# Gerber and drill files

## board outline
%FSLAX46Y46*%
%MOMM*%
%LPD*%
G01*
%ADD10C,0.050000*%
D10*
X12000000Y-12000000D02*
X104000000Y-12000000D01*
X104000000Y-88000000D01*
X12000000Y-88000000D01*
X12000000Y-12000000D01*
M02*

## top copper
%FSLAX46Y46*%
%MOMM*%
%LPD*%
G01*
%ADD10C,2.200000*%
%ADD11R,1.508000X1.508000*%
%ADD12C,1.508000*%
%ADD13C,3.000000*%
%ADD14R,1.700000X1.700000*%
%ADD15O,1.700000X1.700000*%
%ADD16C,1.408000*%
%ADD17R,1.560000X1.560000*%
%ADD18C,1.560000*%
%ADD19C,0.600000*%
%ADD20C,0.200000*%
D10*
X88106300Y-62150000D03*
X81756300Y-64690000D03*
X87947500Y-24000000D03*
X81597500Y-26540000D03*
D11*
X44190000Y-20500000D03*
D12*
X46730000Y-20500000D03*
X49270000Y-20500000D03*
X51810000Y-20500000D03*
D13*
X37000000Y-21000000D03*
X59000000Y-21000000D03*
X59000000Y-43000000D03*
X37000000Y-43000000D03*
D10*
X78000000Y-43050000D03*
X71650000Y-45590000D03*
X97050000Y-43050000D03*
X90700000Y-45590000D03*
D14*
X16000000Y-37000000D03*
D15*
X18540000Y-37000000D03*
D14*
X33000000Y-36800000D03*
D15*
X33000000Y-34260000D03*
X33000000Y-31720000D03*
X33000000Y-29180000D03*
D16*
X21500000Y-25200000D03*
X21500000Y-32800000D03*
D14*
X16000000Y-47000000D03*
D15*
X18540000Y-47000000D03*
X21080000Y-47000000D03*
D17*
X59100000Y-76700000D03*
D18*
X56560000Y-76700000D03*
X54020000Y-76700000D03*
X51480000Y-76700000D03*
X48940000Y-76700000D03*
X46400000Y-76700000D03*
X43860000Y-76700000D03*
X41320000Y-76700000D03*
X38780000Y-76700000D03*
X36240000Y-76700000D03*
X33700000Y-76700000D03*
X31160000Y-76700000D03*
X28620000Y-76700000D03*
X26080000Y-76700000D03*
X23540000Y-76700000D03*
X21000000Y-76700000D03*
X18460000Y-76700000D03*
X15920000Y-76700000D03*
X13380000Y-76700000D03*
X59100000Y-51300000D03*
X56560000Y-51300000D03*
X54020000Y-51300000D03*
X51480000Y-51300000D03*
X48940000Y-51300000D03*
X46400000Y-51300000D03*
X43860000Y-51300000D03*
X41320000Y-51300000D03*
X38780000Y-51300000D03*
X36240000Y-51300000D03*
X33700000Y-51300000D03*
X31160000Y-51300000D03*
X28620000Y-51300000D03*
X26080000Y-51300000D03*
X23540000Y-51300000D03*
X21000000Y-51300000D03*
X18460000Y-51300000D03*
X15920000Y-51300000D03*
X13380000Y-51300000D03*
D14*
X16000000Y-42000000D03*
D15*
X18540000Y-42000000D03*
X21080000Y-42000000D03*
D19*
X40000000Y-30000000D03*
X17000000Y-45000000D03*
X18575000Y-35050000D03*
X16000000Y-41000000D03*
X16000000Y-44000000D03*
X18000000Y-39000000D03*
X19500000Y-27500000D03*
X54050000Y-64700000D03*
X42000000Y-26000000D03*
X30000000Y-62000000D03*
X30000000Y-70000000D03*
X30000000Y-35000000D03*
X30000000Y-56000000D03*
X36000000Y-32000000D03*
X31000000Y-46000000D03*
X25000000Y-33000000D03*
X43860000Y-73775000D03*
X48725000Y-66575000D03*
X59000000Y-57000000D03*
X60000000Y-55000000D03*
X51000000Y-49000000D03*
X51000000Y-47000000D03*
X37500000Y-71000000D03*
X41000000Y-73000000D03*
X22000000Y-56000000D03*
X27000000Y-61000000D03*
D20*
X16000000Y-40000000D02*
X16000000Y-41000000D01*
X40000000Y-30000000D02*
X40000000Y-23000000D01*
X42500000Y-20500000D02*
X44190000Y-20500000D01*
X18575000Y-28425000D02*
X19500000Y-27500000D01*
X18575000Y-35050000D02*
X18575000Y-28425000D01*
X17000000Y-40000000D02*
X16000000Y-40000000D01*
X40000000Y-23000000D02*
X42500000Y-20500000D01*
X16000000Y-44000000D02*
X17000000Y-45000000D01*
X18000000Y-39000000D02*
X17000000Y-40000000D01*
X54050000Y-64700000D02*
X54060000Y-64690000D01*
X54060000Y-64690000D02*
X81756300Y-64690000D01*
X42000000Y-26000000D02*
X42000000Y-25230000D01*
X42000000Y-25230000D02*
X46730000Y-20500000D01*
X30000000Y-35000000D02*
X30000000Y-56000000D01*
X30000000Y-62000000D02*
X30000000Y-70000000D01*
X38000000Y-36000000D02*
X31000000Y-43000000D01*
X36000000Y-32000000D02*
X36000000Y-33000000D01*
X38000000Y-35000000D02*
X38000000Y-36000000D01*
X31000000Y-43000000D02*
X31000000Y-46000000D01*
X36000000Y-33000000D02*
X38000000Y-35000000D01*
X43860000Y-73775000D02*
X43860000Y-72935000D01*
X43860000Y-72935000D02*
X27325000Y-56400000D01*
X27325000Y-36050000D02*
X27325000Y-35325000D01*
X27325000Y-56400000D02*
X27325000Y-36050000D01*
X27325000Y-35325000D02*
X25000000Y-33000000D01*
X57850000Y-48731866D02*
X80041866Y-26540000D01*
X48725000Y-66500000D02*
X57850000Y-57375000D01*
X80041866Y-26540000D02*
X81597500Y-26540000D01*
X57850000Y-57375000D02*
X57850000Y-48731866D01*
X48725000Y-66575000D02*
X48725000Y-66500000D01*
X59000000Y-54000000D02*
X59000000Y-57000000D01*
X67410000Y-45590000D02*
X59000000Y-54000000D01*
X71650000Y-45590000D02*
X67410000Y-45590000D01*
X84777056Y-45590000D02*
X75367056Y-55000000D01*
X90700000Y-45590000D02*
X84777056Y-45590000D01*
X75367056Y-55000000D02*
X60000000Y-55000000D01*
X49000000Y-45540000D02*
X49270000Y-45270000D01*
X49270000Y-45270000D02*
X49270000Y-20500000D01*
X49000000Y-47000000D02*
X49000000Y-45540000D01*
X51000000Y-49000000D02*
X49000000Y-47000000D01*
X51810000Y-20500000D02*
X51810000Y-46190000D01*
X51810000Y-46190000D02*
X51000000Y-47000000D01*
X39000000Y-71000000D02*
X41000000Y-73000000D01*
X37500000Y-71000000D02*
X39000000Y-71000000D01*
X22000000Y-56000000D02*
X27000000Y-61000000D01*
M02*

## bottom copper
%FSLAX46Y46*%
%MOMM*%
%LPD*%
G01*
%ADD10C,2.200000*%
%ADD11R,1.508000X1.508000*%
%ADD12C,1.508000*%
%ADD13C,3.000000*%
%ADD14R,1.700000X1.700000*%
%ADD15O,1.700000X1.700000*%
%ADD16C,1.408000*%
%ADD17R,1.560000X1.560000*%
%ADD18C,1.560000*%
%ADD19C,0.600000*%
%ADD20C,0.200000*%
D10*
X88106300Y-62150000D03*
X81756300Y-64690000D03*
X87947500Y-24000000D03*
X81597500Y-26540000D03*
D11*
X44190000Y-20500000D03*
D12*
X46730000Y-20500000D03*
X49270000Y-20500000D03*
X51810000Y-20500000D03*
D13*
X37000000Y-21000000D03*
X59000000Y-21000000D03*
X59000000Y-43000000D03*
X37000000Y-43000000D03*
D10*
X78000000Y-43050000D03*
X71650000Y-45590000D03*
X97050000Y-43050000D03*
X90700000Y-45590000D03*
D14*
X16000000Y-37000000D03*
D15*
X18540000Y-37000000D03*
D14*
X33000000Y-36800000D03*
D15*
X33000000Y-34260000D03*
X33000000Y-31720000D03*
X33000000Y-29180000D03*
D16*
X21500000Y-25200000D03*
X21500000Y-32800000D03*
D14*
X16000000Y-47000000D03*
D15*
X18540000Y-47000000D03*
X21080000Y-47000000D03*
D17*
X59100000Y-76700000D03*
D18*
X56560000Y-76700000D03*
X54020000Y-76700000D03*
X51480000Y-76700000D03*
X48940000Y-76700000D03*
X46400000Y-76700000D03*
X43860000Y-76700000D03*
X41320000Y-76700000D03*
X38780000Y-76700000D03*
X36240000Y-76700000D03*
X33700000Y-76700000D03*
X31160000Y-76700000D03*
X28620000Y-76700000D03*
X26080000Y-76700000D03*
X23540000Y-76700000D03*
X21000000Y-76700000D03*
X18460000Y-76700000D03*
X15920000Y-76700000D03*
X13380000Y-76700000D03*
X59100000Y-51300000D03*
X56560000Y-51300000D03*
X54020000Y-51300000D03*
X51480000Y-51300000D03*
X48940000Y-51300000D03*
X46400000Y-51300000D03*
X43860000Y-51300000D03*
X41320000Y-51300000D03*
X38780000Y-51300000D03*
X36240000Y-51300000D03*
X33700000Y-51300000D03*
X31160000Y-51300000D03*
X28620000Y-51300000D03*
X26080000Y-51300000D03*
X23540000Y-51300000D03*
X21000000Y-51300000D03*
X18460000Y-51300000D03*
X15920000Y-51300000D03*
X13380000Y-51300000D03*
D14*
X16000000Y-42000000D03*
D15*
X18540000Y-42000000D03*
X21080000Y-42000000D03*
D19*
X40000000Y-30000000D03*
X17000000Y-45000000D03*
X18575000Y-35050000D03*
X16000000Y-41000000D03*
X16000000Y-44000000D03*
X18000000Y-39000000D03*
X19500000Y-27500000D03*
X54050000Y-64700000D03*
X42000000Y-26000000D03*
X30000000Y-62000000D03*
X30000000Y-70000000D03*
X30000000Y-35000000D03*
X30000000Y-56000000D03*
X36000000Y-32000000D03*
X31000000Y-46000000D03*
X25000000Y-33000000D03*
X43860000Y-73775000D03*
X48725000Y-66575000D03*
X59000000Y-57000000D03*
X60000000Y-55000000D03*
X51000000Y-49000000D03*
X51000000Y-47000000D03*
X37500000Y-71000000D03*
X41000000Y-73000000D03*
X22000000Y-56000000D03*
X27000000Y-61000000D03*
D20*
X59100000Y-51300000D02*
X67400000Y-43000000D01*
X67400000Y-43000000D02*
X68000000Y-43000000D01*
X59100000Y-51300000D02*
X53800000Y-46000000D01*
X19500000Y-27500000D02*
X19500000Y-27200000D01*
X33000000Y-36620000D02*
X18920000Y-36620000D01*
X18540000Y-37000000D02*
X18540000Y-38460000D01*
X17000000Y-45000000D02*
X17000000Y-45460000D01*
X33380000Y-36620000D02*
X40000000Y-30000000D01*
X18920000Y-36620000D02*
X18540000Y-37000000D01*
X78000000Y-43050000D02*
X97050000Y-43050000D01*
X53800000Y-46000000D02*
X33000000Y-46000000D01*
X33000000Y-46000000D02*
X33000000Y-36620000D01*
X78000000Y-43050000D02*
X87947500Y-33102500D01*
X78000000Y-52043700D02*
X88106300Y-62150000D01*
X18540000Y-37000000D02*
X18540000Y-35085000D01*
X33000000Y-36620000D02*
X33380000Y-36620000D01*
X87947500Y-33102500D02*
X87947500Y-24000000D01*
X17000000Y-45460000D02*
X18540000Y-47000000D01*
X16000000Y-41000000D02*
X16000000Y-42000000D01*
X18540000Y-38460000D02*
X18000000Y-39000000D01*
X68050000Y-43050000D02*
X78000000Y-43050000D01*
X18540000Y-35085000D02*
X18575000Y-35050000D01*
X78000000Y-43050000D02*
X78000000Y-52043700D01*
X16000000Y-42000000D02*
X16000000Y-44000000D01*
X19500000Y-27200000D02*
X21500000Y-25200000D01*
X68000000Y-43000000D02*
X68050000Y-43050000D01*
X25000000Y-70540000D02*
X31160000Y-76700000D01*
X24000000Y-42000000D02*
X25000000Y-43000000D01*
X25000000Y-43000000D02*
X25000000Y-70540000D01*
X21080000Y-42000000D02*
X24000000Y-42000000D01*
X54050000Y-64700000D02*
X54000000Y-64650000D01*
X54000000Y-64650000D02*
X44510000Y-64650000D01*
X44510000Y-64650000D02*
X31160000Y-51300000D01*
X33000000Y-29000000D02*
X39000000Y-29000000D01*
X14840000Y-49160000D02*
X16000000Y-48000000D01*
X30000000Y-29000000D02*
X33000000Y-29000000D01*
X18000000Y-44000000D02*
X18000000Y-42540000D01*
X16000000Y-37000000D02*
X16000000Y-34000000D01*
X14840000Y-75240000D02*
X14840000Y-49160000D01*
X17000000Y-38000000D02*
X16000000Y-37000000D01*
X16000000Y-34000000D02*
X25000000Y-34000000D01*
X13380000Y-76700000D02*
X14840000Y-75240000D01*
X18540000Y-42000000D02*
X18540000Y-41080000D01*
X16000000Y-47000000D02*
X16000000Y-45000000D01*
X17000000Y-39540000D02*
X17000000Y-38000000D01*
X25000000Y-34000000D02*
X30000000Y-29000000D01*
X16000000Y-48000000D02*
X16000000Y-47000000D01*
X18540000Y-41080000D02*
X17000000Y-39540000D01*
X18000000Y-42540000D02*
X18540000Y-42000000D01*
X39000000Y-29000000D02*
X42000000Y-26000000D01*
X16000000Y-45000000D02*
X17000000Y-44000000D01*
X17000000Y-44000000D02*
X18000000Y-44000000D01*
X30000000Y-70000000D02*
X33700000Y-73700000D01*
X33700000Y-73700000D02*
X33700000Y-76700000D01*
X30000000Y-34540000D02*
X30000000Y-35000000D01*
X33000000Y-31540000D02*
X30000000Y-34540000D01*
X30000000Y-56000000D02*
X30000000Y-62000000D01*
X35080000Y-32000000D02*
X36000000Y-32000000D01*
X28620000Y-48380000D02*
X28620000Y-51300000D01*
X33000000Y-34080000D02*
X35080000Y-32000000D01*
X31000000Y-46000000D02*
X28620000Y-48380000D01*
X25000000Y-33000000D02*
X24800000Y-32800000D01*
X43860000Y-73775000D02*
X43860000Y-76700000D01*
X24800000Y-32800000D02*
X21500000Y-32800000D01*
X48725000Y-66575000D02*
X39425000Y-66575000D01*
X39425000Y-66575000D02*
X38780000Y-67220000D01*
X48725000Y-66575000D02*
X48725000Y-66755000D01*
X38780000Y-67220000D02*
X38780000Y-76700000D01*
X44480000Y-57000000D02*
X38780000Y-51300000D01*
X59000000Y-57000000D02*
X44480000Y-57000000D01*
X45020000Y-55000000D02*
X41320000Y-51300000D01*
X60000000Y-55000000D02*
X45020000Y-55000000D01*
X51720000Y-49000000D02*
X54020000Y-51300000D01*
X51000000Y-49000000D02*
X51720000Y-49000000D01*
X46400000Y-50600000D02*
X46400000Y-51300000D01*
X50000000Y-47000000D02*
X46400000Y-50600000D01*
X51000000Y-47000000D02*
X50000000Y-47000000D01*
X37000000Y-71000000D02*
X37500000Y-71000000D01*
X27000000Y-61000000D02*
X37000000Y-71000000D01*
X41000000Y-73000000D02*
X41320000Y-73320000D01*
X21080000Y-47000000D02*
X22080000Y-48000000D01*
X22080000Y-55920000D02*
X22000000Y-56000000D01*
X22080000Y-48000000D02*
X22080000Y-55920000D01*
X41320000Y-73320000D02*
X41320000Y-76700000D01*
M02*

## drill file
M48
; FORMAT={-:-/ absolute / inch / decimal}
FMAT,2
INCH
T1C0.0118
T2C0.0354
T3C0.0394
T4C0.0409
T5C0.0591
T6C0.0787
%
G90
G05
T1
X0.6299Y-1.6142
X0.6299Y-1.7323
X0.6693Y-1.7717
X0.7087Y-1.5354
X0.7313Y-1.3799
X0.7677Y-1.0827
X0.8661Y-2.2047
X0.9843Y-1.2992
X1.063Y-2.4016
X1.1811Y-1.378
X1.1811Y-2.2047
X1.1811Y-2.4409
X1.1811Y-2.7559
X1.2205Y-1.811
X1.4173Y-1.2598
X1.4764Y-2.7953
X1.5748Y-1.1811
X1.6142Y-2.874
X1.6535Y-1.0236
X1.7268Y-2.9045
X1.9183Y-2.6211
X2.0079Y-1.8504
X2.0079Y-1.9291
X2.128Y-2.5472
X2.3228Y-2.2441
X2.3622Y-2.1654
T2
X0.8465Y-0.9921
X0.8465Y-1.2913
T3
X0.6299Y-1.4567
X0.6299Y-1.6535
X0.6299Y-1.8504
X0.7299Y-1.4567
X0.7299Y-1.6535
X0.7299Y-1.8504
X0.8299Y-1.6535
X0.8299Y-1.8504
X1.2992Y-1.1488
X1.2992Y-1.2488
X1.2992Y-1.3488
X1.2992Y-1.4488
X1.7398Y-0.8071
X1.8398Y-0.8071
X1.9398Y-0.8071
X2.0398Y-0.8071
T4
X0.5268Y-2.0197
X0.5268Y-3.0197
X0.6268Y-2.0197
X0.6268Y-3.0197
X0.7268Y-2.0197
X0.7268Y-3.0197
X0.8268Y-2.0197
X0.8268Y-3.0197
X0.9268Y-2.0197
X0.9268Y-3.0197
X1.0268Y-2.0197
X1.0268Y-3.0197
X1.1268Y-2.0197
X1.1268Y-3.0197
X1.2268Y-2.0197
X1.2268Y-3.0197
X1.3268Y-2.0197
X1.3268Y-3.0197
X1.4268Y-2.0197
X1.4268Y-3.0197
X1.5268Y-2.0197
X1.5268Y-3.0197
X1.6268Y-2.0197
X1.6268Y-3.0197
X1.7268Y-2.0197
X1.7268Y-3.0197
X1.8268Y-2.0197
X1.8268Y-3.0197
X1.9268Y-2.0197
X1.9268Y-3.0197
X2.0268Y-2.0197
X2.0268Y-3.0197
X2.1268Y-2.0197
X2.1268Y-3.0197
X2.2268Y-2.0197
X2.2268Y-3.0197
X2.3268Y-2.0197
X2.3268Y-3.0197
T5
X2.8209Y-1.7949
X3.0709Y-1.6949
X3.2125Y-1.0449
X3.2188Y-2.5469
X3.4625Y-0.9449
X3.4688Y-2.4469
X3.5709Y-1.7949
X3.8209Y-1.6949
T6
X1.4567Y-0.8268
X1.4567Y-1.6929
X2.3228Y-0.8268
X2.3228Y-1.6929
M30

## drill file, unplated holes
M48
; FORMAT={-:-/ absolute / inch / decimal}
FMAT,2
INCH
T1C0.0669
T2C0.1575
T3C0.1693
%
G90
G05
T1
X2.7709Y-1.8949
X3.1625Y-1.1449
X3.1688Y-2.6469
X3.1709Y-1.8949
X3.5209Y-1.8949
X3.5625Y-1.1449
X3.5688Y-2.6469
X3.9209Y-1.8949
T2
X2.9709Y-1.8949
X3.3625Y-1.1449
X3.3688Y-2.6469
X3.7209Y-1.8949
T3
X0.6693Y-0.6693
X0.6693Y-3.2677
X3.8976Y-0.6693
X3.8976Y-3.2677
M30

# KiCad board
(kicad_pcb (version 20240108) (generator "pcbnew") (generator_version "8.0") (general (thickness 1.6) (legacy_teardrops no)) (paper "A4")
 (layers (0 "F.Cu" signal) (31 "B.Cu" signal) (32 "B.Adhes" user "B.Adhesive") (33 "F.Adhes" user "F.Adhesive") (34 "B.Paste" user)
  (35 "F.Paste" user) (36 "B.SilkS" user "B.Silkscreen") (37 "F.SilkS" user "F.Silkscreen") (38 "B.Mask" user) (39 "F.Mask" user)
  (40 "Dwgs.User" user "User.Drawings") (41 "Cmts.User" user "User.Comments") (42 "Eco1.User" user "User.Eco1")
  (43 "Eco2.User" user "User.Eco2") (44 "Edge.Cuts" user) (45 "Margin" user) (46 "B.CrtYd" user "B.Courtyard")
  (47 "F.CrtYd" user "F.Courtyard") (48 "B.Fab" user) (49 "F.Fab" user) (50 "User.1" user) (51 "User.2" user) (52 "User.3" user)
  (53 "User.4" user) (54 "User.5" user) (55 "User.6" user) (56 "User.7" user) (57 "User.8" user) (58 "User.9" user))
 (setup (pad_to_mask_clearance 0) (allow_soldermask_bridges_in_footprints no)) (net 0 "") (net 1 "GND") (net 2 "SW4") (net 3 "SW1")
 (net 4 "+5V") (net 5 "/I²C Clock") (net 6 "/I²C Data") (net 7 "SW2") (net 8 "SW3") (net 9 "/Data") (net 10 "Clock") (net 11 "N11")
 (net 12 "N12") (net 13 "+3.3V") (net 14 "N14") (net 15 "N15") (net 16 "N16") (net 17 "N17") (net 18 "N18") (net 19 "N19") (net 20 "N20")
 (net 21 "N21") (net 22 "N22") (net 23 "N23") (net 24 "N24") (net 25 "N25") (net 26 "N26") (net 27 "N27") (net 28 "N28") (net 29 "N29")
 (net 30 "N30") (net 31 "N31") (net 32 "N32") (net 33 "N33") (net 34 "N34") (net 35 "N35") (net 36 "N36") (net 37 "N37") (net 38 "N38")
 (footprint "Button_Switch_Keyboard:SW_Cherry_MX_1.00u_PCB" (layer "F.Cu") (at 88.1063 62.15)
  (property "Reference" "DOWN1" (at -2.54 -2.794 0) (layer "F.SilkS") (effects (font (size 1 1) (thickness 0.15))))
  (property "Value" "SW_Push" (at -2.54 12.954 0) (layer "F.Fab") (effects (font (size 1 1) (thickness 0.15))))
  (pad "" np_thru_hole circle (at -7.62 5.08) (size 1.7 1.7) (drill 1.7) (layers "*.Cu" "*.Mask"))
  (pad "" np_thru_hole circle (at -2.54 5.08) (size 4 4) (drill 4) (layers "*.Cu" "*.Mask"))
  (pad "" np_thru_hole circle (at 2.54 5.08) (size 1.7 1.7) (drill 1.7) (layers "*.Cu" "*.Mask"))
  (pad "1" thru_hole circle (at 0 0) (size 2.2 2.2) (drill 1.5) (layers "*.Cu" "*.Mask") (remove_unused_layers no) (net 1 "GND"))
  (pad "2" thru_hole circle (at -6.35 2.54) (size 2.2 2.2) (drill 1.5) (layers "*.Cu" "*.Mask") (remove_unused_layers no) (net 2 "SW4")))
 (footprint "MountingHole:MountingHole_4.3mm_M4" (layer "F.Cu") (at 99 17)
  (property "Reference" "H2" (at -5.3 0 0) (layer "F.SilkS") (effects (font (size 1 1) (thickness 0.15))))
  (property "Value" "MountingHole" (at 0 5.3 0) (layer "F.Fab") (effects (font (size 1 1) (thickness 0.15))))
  (pad "" np_thru_hole circle (at 0 0) (size 4.3 4.3) (drill 4.3) (layers "*.Cu" "*.Mask")))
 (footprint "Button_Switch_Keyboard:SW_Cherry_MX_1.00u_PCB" (layer "F.Cu") (at 87.9475 24)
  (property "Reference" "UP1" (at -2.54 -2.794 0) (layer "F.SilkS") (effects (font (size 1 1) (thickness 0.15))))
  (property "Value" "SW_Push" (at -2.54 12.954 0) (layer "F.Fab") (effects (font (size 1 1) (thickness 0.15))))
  (pad "" np_thru_hole circle (at -7.62 5.08) (size 1.7 1.7) (drill 1.7) (layers "*.Cu" "*.Mask"))
  (pad "" np_thru_hole circle (at -2.54 5.08) (size 4 4) (drill 4) (layers "*.Cu" "*.Mask"))
  (pad "" np_thru_hole circle (at 2.54 5.08) (size 1.7 1.7) (drill 1.7) (layers "*.Cu" "*.Mask"))
  (pad "1" thru_hole circle (at 0 0) (size 2.2 2.2) (drill 1.5) (layers "*.Cu" "*.Mask") (remove_unused_layers no) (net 1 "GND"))
  (pad "2" thru_hole circle (at -6.35 2.54) (size 2.2 2.2) (drill 1.5) (layers "*.Cu" "*.Mask") (remove_unused_layers no) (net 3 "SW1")))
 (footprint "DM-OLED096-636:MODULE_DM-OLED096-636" (layer "F.Cu") (at 48 32)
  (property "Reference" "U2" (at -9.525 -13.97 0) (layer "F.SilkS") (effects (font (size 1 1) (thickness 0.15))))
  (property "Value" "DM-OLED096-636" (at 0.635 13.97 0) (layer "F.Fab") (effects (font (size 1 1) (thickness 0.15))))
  (pad "1" thru_hole rect (at -3.81 -11.5) (size 1.508 1.508) (drill 1) (layers "*.Cu" "*.Mask") (remove_unused_layers no) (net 1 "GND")
   (solder_mask_margin 0.102))
  (pad "2" thru_hole circle (at -1.27 -11.5) (size 1.508 1.508) (drill 1) (layers "*.Cu" "*.Mask") (remove_unused_layers no) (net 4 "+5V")
   (solder_mask_margin 0.102))
  (pad "3" thru_hole circle (at 1.27 -11.5) (size 1.508 1.508) (drill 1) (layers "*.Cu" "*.Mask") (remove_unused_layers no)
   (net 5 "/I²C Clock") (solder_mask_margin 0.102))
  (pad "4" thru_hole circle (at 3.81 -11.5) (size 1.508 1.508) (drill 1) (layers "*.Cu" "*.Mask") (remove_unused_layers no)
   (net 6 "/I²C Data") (solder_mask_margin 0.102))
  (pad "S1" thru_hole circle (at -11 -11) (size 3 3) (drill 2) (layers "*.Cu" "*.Mask") (remove_unused_layers no) (solder_mask_margin 0.102))
  (pad "S2" thru_hole circle (at 11 -11) (size 3 3) (drill 2) (layers "*.Cu" "*.Mask") (remove_unused_layers no) (solder_mask_margin 0.102))
  (pad "S3" thru_hole circle (at 11 11) (size 3 3) (drill 2) (layers "*.Cu" "*.Mask") (remove_unused_layers no) (solder_mask_margin 0.102))
  (pad "S4" thru_hole circle (at -11 11) (size 3 3) (drill 2) (layers "*.Cu" "*.Mask") (remove_unused_layers no) (solder_mask_margin 0.102)))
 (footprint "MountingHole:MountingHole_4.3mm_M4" (layer "F.Cu") (at 99 83)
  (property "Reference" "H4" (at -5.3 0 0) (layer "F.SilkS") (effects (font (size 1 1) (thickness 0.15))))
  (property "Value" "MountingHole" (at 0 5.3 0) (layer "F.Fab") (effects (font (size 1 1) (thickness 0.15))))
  (pad "" np_thru_hole circle (at 0 0) (size 4.3 4.3) (drill 4.3) (layers "*.Cu" "*.Mask")))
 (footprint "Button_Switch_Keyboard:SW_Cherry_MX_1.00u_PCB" (layer "F.Cu") (at 78 43.05)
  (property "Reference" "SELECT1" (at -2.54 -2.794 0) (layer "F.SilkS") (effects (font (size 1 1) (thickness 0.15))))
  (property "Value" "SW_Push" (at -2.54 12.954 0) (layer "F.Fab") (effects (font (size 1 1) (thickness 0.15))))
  (pad "" np_thru_hole circle (at -7.62 5.08) (size 1.7 1.7) (drill 1.7) (layers "*.Cu" "*.Mask"))
  (pad "" np_thru_hole circle (at -2.54 5.08) (size 4 4) (drill 4) (layers "*.Cu" "*.Mask"))
  (pad "" np_thru_hole circle (at 2.54 5.08) (size 1.7 1.7) (drill 1.7) (layers "*.Cu" "*.Mask"))
  (pad "1" thru_hole circle (at 0 0) (size 2.2 2.2) (drill 1.5) (layers "*.Cu" "*.Mask") (remove_unused_layers no) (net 1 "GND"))
  (pad "2" thru_hole circle (at -6.35 2.54) (size 2.2 2.2) (drill 1.5) (layers "*.Cu" "*.Mask") (remove_unused_layers no) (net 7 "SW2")))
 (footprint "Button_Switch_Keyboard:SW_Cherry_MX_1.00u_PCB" (layer "F.Cu") (at 97.05 43.05)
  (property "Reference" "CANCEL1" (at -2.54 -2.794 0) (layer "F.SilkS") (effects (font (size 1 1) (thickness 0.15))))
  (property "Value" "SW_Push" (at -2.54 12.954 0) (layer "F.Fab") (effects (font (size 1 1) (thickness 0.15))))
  (pad "" np_thru_hole circle (at -7.62 5.08) (size 1.7 1.7) (drill 1.7) (layers "*.Cu" "*.Mask"))
  (pad "" np_thru_hole circle (at -2.54 5.08) (size 4 4) (drill 4) (layers "*.Cu" "*.Mask"))
  (pad "" np_thru_hole circle (at 2.54 5.08) (size 1.7 1.7) (drill 1.7) (layers "*.Cu" "*.Mask"))
  (pad "1" thru_hole circle (at 0 0) (size 2.2 2.2) (drill 1.5) (layers "*.Cu" "*.Mask") (remove_unused_layers no) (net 1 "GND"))
  (pad "2" thru_hole circle (at -6.35 2.54) (size 2.2 2.2) (drill 1.5) (layers "*.Cu" "*.Mask") (remove_unused_layers no) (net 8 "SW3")))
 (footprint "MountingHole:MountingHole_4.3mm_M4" (layer "F.Cu") (at 17 17)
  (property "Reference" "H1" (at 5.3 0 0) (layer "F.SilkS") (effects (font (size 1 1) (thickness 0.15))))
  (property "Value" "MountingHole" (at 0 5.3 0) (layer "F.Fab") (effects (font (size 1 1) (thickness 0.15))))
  (pad "" np_thru_hole circle (at 0 0) (size 4.3 4.3) (drill 4.3) (layers "*.Cu" "*.Mask")))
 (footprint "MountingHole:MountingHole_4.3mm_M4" (layer "F.Cu") (at 17 83)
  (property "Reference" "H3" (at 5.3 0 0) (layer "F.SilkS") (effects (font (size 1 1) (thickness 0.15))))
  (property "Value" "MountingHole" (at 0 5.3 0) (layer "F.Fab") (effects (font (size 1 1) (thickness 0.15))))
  (pad "" np_thru_hole circle (at 0 0) (size 4.3 4.3) (drill 4.3) (layers "*.Cu" "*.Mask")))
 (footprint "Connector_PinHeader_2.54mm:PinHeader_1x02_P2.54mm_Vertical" (layer "B.Cu") (at 16 37 -90)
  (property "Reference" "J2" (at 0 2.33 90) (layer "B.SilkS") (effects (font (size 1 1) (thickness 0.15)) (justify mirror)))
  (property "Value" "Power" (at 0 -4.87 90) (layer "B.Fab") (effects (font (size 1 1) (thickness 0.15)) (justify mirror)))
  (pad "1" thru_hole rect (at 0 0 270) (size 1.7 1.7) (drill 1) (layers "*.Cu" "*.Mask") (remove_unused_layers no) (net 4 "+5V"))
  (pad "2" thru_hole oval (at 0 -2.54 270) (size 1.7 1.7) (drill 1) (layers "*.Cu" "*.Mask") (remove_unused_layers no) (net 1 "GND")))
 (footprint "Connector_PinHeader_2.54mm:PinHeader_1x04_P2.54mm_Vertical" (layer "B.Cu") (at 33 36.8)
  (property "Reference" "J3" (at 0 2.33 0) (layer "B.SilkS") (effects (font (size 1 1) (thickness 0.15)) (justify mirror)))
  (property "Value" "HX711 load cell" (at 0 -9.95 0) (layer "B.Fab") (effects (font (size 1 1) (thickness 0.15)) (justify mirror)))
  (pad "1" thru_hole rect (at 0 0) (size 1.7 1.7) (drill 1) (layers "*.Cu" "*.Mask") (remove_unused_layers no) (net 1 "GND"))
  (pad "2" thru_hole oval (at 0 -2.54) (size 1.7 1.7) (drill 1) (layers "*.Cu" "*.Mask") (remove_unused_layers no) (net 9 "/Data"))
  (pad "3" thru_hole oval (at 0 -5.08) (size 1.7 1.7) (drill 1) (layers "*.Cu" "*.Mask") (remove_unused_layers no) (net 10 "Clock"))
  (pad "4" thru_hole oval (at 0 -7.62) (size 1.7 1.7) (drill 1) (layers "*.Cu" "*.Mask") (remove_unused_layers no) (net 4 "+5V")))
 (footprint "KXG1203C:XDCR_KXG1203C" (layer "B.Cu") (at 21.5 29 90)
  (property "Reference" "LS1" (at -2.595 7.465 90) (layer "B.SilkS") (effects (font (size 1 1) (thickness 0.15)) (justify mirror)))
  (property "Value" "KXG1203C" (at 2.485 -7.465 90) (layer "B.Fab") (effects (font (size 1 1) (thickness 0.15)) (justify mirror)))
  (pad "N" thru_hole circle (at 3.8 0 90) (size 1.408 1.408) (drill 0.9) (layers "*.Cu" "*.Mask") (remove_unused_layers no) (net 1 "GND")
   (solder_mask_margin 0.102))
  (pad "P" thru_hole circle (at -3.8 0 90) (size 1.408 1.408) (drill 0.9) (layers "*.Cu" "*.Mask") (remove_unused_layers no) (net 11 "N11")
   (solder_mask_margin 0.102)))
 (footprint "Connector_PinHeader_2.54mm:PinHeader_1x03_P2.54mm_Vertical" (layer "B.Cu") (at 16 47 -90)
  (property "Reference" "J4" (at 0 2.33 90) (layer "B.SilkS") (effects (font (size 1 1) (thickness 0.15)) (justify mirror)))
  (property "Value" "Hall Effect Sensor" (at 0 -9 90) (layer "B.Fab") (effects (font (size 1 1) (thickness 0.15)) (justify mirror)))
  (pad "1" thru_hole rect (at 0 0 270) (size 1.7 1.7) (drill 1) (layers "*.Cu" "*.Mask") (remove_unused_layers no) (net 4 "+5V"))
  (pad "2" thru_hole oval (at 0 -2.54 270) (size 1.7 1.7) (drill 1) (layers "*.Cu" "*.Mask") (remove_unused_layers no) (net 1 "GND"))
  (pad "3" thru_hole oval (at 0 -5.08 270) (size 1.7 1.7) (drill 1) (layers "*.Cu" "*.Mask") (remove_unused_layers no) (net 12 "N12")))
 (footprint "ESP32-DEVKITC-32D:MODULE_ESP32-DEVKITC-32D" (layer "B.Cu") (at 39.34 64 90)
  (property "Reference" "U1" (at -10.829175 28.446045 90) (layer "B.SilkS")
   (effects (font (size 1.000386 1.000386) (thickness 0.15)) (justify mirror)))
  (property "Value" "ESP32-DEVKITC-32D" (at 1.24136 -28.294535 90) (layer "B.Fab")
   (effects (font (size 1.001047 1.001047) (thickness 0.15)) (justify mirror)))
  (pad "J2-1" thru_hole rect (at -12.7 19.76 90) (size 1.56 1.56) (drill 1.04) (layers "*.Cu" "*.Mask") (remove_unused_layers no)
   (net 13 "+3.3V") (solder_mask_margin 0.102))
  (pad "J2-2" thru_hole circle (at -12.7 17.22 90) (size 1.56 1.56) (drill 1.04) (layers "*.Cu" "*.Mask") (remove_unused_layers no)
   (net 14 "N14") (solder_mask_margin 0.102))
  (pad "J2-3" thru_hole circle (at -12.7 14.68 90) (size 1.56 1.56) (drill 1.04) (layers "*.Cu" "*.Mask") (remove_unused_layers no)
   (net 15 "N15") (solder_mask_margin 0.102))
  (pad "J2-4" thru_hole circle (at -12.7 12.14 90) (size 1.56 1.56) (drill 1.04) (layers "*.Cu" "*.Mask") (remove_unused_layers no)
   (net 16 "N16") (solder_mask_margin 0.102))
  (pad "J2-5" thru_hole circle (at -12.7 9.6 90) (size 1.56 1.56) (drill 1.04) (layers "*.Cu" "*.Mask") (remove_unused_layers no)
   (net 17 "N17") (solder_mask_margin 0.102))
  (pad "J2-6" thru_hole circle (at -12.7 7.06 90) (size 1.56 1.56) (drill 1.04) (layers "*.Cu" "*.Mask") (remove_unused_layers no)
   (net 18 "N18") (solder_mask_margin 0.102))
  (pad "J2-7" thru_hole circle (at -12.7 4.52 90) (size 1.56 1.56) (drill 1.04) (layers "*.Cu" "*.Mask") (remove_unused_layers no)
   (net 11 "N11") (solder_mask_margin 0.102))
  (pad "J2-8" thru_hole circle (at -12.7 1.98 90) (size 1.56 1.56) (drill 1.04) (layers "*.Cu" "*.Mask") (remove_unused_layers no)
   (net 12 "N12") (solder_mask_margin 0.102))
  (pad "J2-9" thru_hole circle (at -12.7 -0.56 90) (size 1.56 1.56) (drill 1.04) (layers "*.Cu" "*.Mask") (remove_unused_layers no)
   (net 3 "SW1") (solder_mask_margin 0.102))
  (pad "J2-10" thru_hole circle (at -12.7 -3.1 90) (size 1.56 1.56) (drill 1.04) (layers "*.Cu" "*.Mask") (remove_unused_layers no)
   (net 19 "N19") (solder_mask_margin 0.102))
  (pad "J2-11" thru_hole circle (at -12.7 -5.64 90) (size 1.56 1.56) (drill 1.04) (layers "*.Cu" "*.Mask") (remove_unused_layers no)
   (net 10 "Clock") (solder_mask_margin 0.102))
  (pad "J2-12" thru_hole circle (at -12.7 -8.18 90) (size 1.56 1.56) (drill 1.04) (layers "*.Cu" "*.Mask") (remove_unused_layers no)
   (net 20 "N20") (solder_mask_margin 0.102))
  (pad "J2-13" thru_hole circle (at -12.7 -10.72 90) (size 1.56 1.56) (drill 1.04) (layers "*.Cu" "*.Mask") (remove_unused_layers no)
   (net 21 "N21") (solder_mask_margin 0.102))
  (pad "J2-14" thru_hole circle (at -12.7 -13.26 90) (size 1.56 1.56) (drill 1.04) (layers "*.Cu" "*.Mask") (remove_unused_layers no)
   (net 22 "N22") (solder_mask_margin 0.102))
  (pad "J2-15" thru_hole circle (at -12.7 -15.8 90) (size 1.56 1.56) (drill 1.04) (layers "*.Cu" "*.Mask") (remove_unused_layers no)
   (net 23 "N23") (solder_mask_margin 0.102))
  (pad "J2-16" thru_hole circle (at -12.7 -18.34 90) (size 1.56 1.56) (drill 1.04) (layers "*.Cu" "*.Mask") (remove_unused_layers no)
   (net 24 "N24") (solder_mask_margin 0.102))
  (pad "J2-17" thru_hole circle (at -12.7 -20.88 90) (size 1.56 1.56) (drill 1.04) (layers "*.Cu" "*.Mask") (remove_unused_layers no)
   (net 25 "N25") (solder_mask_margin 0.102))
  (pad "J2-18" thru_hole circle (at -12.7 -23.42 90) (size 1.56 1.56) (drill 1.04) (layers "*.Cu" "*.Mask") (remove_unused_layers no)
   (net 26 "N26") (solder_mask_margin 0.102))
  (pad "J2-19" thru_hole circle (at -12.7 -25.96 90) (size 1.56 1.56) (drill 1.04) (layers "*.Cu" "*.Mask") (remove_unused_layers no)
   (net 4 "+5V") (solder_mask_margin 0.102))
  (pad "J3-1" thru_hole circle (at 12.7 19.76 90) (size 1.56 1.56) (drill 1.04) (layers "*.Cu" "*.Mask") (remove_unused_layers no)
   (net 1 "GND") (solder_mask_margin 0.102))
  (pad "J3-2" thru_hole circle (at 12.7 17.22 90) (size 1.56 1.56) (drill 1.04) (layers "*.Cu" "*.Mask") (remove_unused_layers no)
   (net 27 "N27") (solder_mask_margin 0.102))
  (pad "J3-3" thru_hole circle (at 12.7 14.68 90) (size 1.56 1.56) (drill 1.04) (layers "*.Cu" "*.Mask") (remove_unused_layers no)
   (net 5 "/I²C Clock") (solder_mask_margin 0.102))
  (pad "J3-4" thru_hole circle (at 12.7 12.14 90) (size 1.56 1.56) (drill 1.04) (layers "*.Cu" "*.Mask") (remove_unused_layers no)
   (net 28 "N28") (solder_mask_margin 0.102))
  (pad "J3-5" thru_hole circle (at 12.7 9.6 90) (size 1.56 1.56) (drill 1.04) (layers "*.Cu" "*.Mask") (remove_unused_layers no)
   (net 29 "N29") (solder_mask_margin 0.102))
  (pad "J3-6" thru_hole circle (at 12.7 7.06 90) (size 1.56 1.56) (drill 1.04) (layers "*.Cu" "*.Mask") (remove_unused_layers no)
   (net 6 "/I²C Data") (solder_mask_margin 0.102))
  (pad "J3-7" thru_hole circle (at 12.7 4.52 90) (size 1.56 1.56) (drill 1.04) (layers "*.Cu" "*.Mask") (remove_unused_layers no)
   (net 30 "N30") (solder_mask_margin 0.102))
  (pad "J3-8" thru_hole circle (at 12.7 1.98 90) (size 1.56 1.56) (drill 1.04) (layers "*.Cu" "*.Mask") (remove_unused_layers no)
   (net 8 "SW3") (solder_mask_margin 0.102))
  (pad "J3-9" thru_hole circle (at 12.7 -0.56 90) (size 1.56 1.56) (drill 1.04) (layers "*.Cu" "*.Mask") (remove_unused_layers no)
   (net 7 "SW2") (solder_mask_margin 0.102))
  (pad "J3-10" thru_hole circle (at 12.7 -3.1 90) (size 1.56 1.56) (drill 1.04) (layers "*.Cu" "*.Mask") (remove_unused_layers no)
   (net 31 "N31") (solder_mask_margin 0.102))
  (pad "J3-11" thru_hole circle (at 12.7 -5.64 90) (size 1.56 1.56) (drill 1.04) (layers "*.Cu" "*.Mask") (remove_unused_layers no)
   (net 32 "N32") (solder_mask_margin 0.102))
  (pad "J3-12" thru_hole circle (at 12.7 -8.18 90) (size 1.56 1.56) (drill 1.04) (layers "*.Cu" "*.Mask") (remove_unused_layers no)
   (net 2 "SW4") (solder_mask_margin 0.102))
  (pad "J3-13" thru_hole circle (at 12.7 -10.72 90) (size 1.56 1.56) (drill 1.04) (layers "*.Cu" "*.Mask") (remove_unused_layers no)
   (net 9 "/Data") (solder_mask_margin 0.102))
  (pad "J3-14" thru_hole circle (at 12.7 -13.26 90) (size 1.56 1.56) (drill 1.04) (layers "*.Cu" "*.Mask") (remove_unused_layers no)
   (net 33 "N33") (solder_mask_margin 0.102))
  (pad "J3-15" thru_hole circle (at 12.7 -15.8 90) (size 1.56 1.56) (drill 1.04) (layers "*.Cu" "*.Mask") (remove_unused_layers no)
   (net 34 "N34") (solder_mask_margin 0.102))
  (pad "J3-16" thru_hole circle (at 12.7 -18.34 90) (size 1.56 1.56) (drill 1.04) (layers "*.Cu" "*.Mask") (remove_unused_layers no)
   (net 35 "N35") (solder_mask_margin 0.102))
  (pad "J3-17" thru_hole circle (at 12.7 -20.88 90) (size 1.56 1.56) (drill 1.04) (layers "*.Cu" "*.Mask") (remove_unused_layers no)
   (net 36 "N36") (solder_mask_margin 0.102))
  (pad "J3-18" thru_hole circle (at 12.7 -23.42 90) (size 1.56 1.56) (drill 1.04) (layers "*.Cu" "*.Mask") (remove_unused_layers no)
   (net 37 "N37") (solder_mask_margin 0.102))
  (pad "J3-19" thru_hole circle (at 12.7 -25.96 90) (size 1.56 1.56) (drill 1.04) (layers "*.Cu" "*.Mask") (remove_unused_layers no)
   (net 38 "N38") (solder_mask_margin 0.102)))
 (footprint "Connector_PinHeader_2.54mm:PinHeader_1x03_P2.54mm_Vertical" (layer "B.Cu") (at 16 42 -90)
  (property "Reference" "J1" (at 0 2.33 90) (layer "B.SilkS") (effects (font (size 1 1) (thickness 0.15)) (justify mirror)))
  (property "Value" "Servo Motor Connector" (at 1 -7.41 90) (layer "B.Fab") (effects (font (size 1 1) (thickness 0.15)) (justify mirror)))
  (pad "1" thru_hole rect (at 0 0 270) (size 1.7 1.7) (drill 1) (layers "*.Cu" "*.Mask") (remove_unused_layers no) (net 1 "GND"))
  (pad "2" thru_hole oval (at 0 -2.54 270) (size 1.7 1.7) (drill 1) (layers "*.Cu" "*.Mask") (remove_unused_layers no) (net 4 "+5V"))
  (pad "3" thru_hole oval (at 0 -5.08 270) (size 1.7 1.7) (drill 1) (layers "*.Cu" "*.Mask") (remove_unused_layers no) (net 20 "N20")))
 (gr_rect (start 12 12) (end 104 88) (stroke (width 0.05) (type default)) (fill none) (layer "Edge.Cuts"))
 (segment (start 16 40) (end 16 41) (width 0.2) (layer "F.Cu") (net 1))
 (segment (start 40 30) (end 40 23) (width 0.2) (layer "F.Cu") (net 1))
 (segment (start 42.5 20.5) (end 44.19 20.5) (width 0.2) (layer "F.Cu") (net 1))
 (segment (start 18.575 28.425) (end 19.5 27.5) (width 0.2) (layer "F.Cu") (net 1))
 (segment (start 18.575 35.05) (end 18.575 28.425) (width 0.2) (layer "F.Cu") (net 1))
 (segment (start 17 40) (end 16 40) (width 0.2) (layer "F.Cu") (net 1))
 (segment (start 40 23) (end 42.5 20.5) (width 0.2) (layer "F.Cu") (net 1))
 (segment (start 16 44) (end 17 45) (width 0.2) (layer "F.Cu") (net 1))
 (segment (start 18 39) (end 17 40) (width 0.2) (layer "F.Cu") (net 1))
 (via (at 40 30) (size 0.6) (drill 0.3) (layers "F.Cu" "B.Cu") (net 1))
 (via (at 17 45) (size 0.6) (drill 0.3) (layers "F.Cu" "B.Cu") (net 1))
 (via (at 18.575 35.05) (size 0.6) (drill 0.3) (layers "F.Cu" "B.Cu") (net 1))
 (via (at 16 41) (size 0.6) (drill 0.3) (layers "F.Cu" "B.Cu") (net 1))
 (via (at 16 44) (size 0.6) (drill 0.3) (layers "F.Cu" "B.Cu") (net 1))
 (via (at 18 39) (size 0.6) (drill 0.3) (layers "F.Cu" "B.Cu") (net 1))
 (via (at 19.5 27.5) (size 0.6) (drill 0.3) (layers "F.Cu" "B.Cu") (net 1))
 (segment (start 59.1 51.3) (end 67.4 43) (width 0.2) (layer "B.Cu") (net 1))
 (segment (start 67.4 43) (end 68 43) (width 0.2) (layer "B.Cu") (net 1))
 (segment (start 59.1 51.3) (end 53.8 46) (width 0.2) (layer "B.Cu") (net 1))
 (segment (start 19.5 27.5) (end 19.5 27.2) (width 0.2) (layer "B.Cu") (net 1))
 (segment (start 33 36.62) (end 18.92 36.62) (width 0.2) (layer "B.Cu") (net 1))
 (segment (start 18.54 37) (end 18.54 38.46) (width 0.2) (layer "B.Cu") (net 1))
 (segment (start 17 45) (end 17 45.46) (width 0.2) (layer "B.Cu") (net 1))
 (segment (start 33.38 36.62) (end 40 30) (width 0.2) (layer "B.Cu") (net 1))
 (segment (start 18.92 36.62) (end 18.54 37) (width 0.2) (layer "B.Cu") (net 1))
 (segment (start 78 43.05) (end 97.05 43.05) (width 0.2) (layer "B.Cu") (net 1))
 (segment (start 53.8 46) (end 33 46) (width 0.2) (layer "B.Cu") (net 1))
 (segment (start 33 46) (end 33 36.62) (width 0.2) (layer "B.Cu") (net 1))
 (segment (start 78 43.05) (end 87.9475 33.1025) (width 0.2) (layer "B.Cu") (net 1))
 (segment (start 78 52.0437) (end 88.1063 62.15) (width 0.2) (layer "B.Cu") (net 1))
 (segment (start 18.54 37) (end 18.54 35.085) (width 0.2) (layer "B.Cu") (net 1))
 (segment (start 33 36.62) (end 33.38 36.62) (width 0.2) (layer "B.Cu") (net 1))
 (segment (start 87.9475 33.1025) (end 87.9475 24) (width 0.2) (layer "B.Cu") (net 1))
 (segment (start 17 45.46) (end 18.54 47) (width 0.2) (layer "B.Cu") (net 1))
 (segment (start 16 41) (end 16 42) (width 0.2) (layer "B.Cu") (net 1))
 (segment (start 18.54 38.46) (end 18 39) (width 0.2) (layer "B.Cu") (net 1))
 (segment (start 68.05 43.05) (end 78 43.05) (width 0.2) (layer "B.Cu") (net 1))
 (segment (start 18.54 35.085) (end 18.575 35.05) (width 0.2) (layer "B.Cu") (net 1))
 (segment (start 78 43.05) (end 78 52.0437) (width 0.2) (layer "B.Cu") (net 1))
 (segment (start 16 42) (end 16 44) (width 0.2) (layer "B.Cu") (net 1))
 (segment (start 19.5 27.2) (end 21.5 25.2) (width 0.2) (layer "B.Cu") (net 1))
 (segment (start 68 43) (end 68.05 43.05) (width 0.2) (layer "B.Cu") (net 1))
 (segment (start 25 70.54) (end 31.16 76.7) (width 0.2) (layer "B.Cu") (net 20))
 (segment (start 24 42) (end 25 43) (width 0.2) (layer "B.Cu") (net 20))
 (segment (start 25 43) (end 25 70.54) (width 0.2) (layer "B.Cu") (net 20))
 (segment (start 21.08 42) (end 24 42) (width 0.2) (layer "B.Cu") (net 20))
 (segment (start 54.05 64.7) (end 54.06 64.69) (width 0.2) (layer "F.Cu") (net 2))
 (segment (start 54.06 64.69) (end 81.7563 64.69) (width 0.2) (layer "F.Cu") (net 2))
 (via (at 54.05 64.7) (size 0.6) (drill 0.3) (layers "F.Cu" "B.Cu") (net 2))
 (segment (start 54.05 64.7) (end 54 64.65) (width 0.2) (layer "B.Cu") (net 2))
 (segment (start 54 64.65) (end 44.51 64.65) (width 0.2) (layer "B.Cu") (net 2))
 (segment (start 44.51 64.65) (end 31.16 51.3) (width 0.2) (layer "B.Cu") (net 2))
 (segment (start 42 26) (end 42 25.23) (width 0.2) (layer "F.Cu") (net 4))
 (segment (start 42 25.23) (end 46.73 20.5) (width 0.2) (layer "F.Cu") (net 4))
 (via (at 42 26) (size 0.6) (drill 0.3) (layers "F.Cu" "B.Cu") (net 4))
 (segment (start 33 29) (end 39 29) (width 0.2) (layer "B.Cu") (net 4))
 (segment (start 14.84 49.16) (end 16 48) (width 0.2) (layer "B.Cu") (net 4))
 (segment (start 30 29) (end 33 29) (width 0.2) (layer "B.Cu") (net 4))
 (segment (start 18 44) (end 18 42.54) (width 0.2) (layer "B.Cu") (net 4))
 (segment (start 16 37) (end 16 34) (width 0.2) (layer "B.Cu") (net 4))
 (segment (start 14.84 75.24) (end 14.84 49.16) (width 0.2) (layer "B.Cu") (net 4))
 (segment (start 17 38) (end 16 37) (width 0.2) (layer "B.Cu") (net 4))
 (segment (start 16 34) (end 25 34) (width 0.2) (layer "B.Cu") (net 4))
 (segment (start 13.38 76.7) (end 14.84 75.24) (width 0.2) (layer "B.Cu") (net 4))
 (segment (start 18.54 42) (end 18.54 41.08) (width 0.2) (layer "B.Cu") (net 4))
 (segment (start 16 47) (end 16 45) (width 0.2) (layer "B.Cu") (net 4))
 (segment (start 17 39.54) (end 17 38) (width 0.2) (layer "B.Cu") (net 4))
 (segment (start 25 34) (end 30 29) (width 0.2) (layer "B.Cu") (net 4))
 (segment (start 16 48) (end 16 47) (width 0.2) (layer "B.Cu") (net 4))
 (segment (start 18.54 41.08) (end 17 39.54) (width 0.2) (layer "B.Cu") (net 4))
 (segment (start 18 42.54) (end 18.54 42) (width 0.2) (layer "B.Cu") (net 4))
 (segment (start 39 29) (end 42 26) (width 0.2) (layer "B.Cu") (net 4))
 (segment (start 16 45) (end 17 44) (width 0.2) (layer "B.Cu") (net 4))
 (segment (start 17 44) (end 18 44) (width 0.2) (layer "B.Cu") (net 4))
 (segment (start 30 35) (end 30 56) (width 0.2) (layer "F.Cu") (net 10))
 (segment (start 30 62) (end 30 70) (width 0.2) (layer "F.Cu") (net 10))
 (via (at 30 62) (size 0.6) (drill 0.3) (layers "F.Cu" "B.Cu") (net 10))
 (via (at 30 70) (size 0.6) (drill 0.3) (layers "F.Cu" "B.Cu") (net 10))
 (via (at 30 35) (size 0.6) (drill 0.3) (layers "F.Cu" "B.Cu") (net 10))
 (via (at 30 56) (size 0.6) (drill 0.3) (layers "F.Cu" "B.Cu") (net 10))
 (segment (start 30 70) (end 33.7 73.7) (width 0.2) (layer "B.Cu") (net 10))
 (segment (start 33.7 73.7) (end 33.7 76.7) (width 0.2) (layer "B.Cu") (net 10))
 (segment (start 30 34.54) (end 30 35) (width 0.2) (layer "B.Cu") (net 10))
 (segment (start 33 31.54) (end 30 34.54) (width 0.2) (layer "B.Cu") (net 10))
 (segment (start 30 56) (end 30 62) (width 0.2) (layer "B.Cu") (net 10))
 (segment (start 38 36) (end 31 43) (width 0.2) (layer "F.Cu") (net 9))
 (segment (start 36 32) (end 36 33) (width 0.2) (layer "F.Cu") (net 9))
 (segment (start 38 35) (end 38 36) (width 0.2) (layer "F.Cu") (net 9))
 (segment (start 31 43) (end 31 46) (width 0.2) (layer "F.Cu") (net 9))
 (segment (start 36 33) (end 38 35) (width 0.2) (layer "F.Cu") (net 9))
 (via (at 36 32) (size 0.6) (drill 0.3) (layers "F.Cu" "B.Cu") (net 9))
 (via (at 31 46) (size 0.6) (drill 0.3) (layers "F.Cu" "B.Cu") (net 9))
 (segment (start 35.08 32) (end 36 32) (width 0.2) (layer "B.Cu") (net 9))
 (segment (start 28.62 48.38) (end 28.62 51.3) (width 0.2) (layer "B.Cu") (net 9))
 (segment (start 33 34.08) (end 35.08 32) (width 0.2) (layer "B.Cu") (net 9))
 (segment (start 31 46) (end 28.62 48.38) (width 0.2) (layer "B.Cu") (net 9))
 (segment (start 43.86 73.775) (end 43.86 72.935) (width 0.2) (layer "F.Cu") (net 11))
 (segment (start 43.86 72.935) (end 27.325 56.4) (width 0.2) (layer "F.Cu") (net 11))
 (segment (start 27.325 36.05) (end 27.325 35.325) (width 0.2) (layer "F.Cu") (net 11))
 (segment (start 27.325 56.4) (end 27.325 36.05) (width 0.2) (layer "F.Cu") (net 11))
 (segment (start 27.325 35.325) (end 25 33) (width 0.2) (layer "F.Cu") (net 11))
 (via (at 25 33) (size 0.6) (drill 0.3) (layers "F.Cu" "B.Cu") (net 11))
 (via (at 43.86 73.775) (size 0.6) (drill 0.3) (layers "F.Cu" "B.Cu") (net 11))
 (segment (start 25 33) (end 24.8 32.8) (width 0.2) (layer "B.Cu") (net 11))
 (segment (start 43.86 73.775) (end 43.86 76.7) (width 0.2) (layer "B.Cu") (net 11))
 (segment (start 24.8 32.8) (end 21.5 32.8) (width 0.2) (layer "B.Cu") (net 11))
 (segment (start 57.85 48.731866) (end 80.041866 26.54) (width 0.2) (layer "F.Cu") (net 3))
 (segment (start 48.725 66.5) (end 57.85 57.375) (width 0.2) (layer "F.Cu") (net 3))
 (segment (start 80.041866 26.54) (end 81.5975 26.54) (width 0.2) (layer "F.Cu") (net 3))
 (segment (start 57.85 57.375) (end 57.85 48.731866) (width 0.2) (layer "F.Cu") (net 3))
 (segment (start 48.725 66.575) (end 48.725 66.5) (width 0.2) (layer "F.Cu") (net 3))
 (via (at 48.725 66.575) (size 0.6) (drill 0.3) (layers "F.Cu" "B.Cu") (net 3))
 (segment (start 48.725 66.575) (end 39.425 66.575) (width 0.2) (layer "B.Cu") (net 3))
 (segment (start 39.425 66.575) (end 38.78 67.22) (width 0.2) (layer "B.Cu") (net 3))
 (segment (start 48.725 66.575) (end 48.725 66.755) (width 0.2) (layer "B.Cu") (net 3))
 (segment (start 38.78 67.22) (end 38.78 76.7) (width 0.2) (layer "B.Cu") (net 3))
 (segment (start 59 54) (end 59 57) (width 0.2) (layer "F.Cu") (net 7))
 (segment (start 67.41 45.59) (end 59 54) (width 0.2) (layer "F.Cu") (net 7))
 (segment (start 71.65 45.59) (end 67.41 45.59) (width 0.2) (layer "F.Cu") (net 7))
 (via (at 59 57) (size 0.6) (drill 0.3) (layers "F.Cu" "B.Cu") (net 7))
 (segment (start 44.48 57) (end 38.78 51.3) (width 0.2) (layer "B.Cu") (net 7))
 (segment (start 59 57) (end 44.48 57) (width 0.2) (layer "B.Cu") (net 7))
 (segment (start 84.777056 45.59) (end 75.367056 55) (width 0.2) (layer "F.Cu") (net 8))
 (segment (start 90.7 45.59) (end 84.777056 45.59) (width 0.2) (layer "F.Cu") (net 8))
 (segment (start 75.367056 55) (end 60 55) (width 0.2) (layer "F.Cu") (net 8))
 (via (at 60 55) (size 0.6) (drill 0.3) (layers "F.Cu" "B.Cu") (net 8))
 (segment (start 45.02 55) (end 41.32 51.3) (width 0.2) (layer "B.Cu") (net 8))
 (segment (start 60 55) (end 45.02 55) (width 0.2) (layer "B.Cu") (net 8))
 (segment (start 49 45.54) (end 49.27 45.27) (width 0.2) (layer "F.Cu") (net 5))
 (segment (start 49.27 45.27) (end 49.27 20.5) (width 0.2) (layer "F.Cu") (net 5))
 (segment (start 49 47) (end 49 45.54) (width 0.2) (layer "F.Cu") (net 5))
 (segment (start 51 49) (end 49 47) (width 0.2) (layer "F.Cu") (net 5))
 (via (at 51 49) (size 0.6) (drill 0.3) (layers "F.Cu" "B.Cu") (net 5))
 (segment (start 51.72 49) (end 54.02 51.3) (width 0.2) (layer "B.Cu") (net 5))
 (segment (start 51 49) (end 51.72 49) (width 0.2) (layer "B.Cu") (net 5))
 (segment (start 51.81 20.5) (end 51.81 46.19) (width 0.2) (layer "F.Cu") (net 6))
 (segment (start 51.81 46.19) (end 51 47) (width 0.2) (layer "F.Cu") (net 6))
 (via (at 51 47) (size 0.6) (drill 0.3) (layers "F.Cu" "B.Cu") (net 6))
 (segment (start 46.4 50.6) (end 46.4 51.3) (width 0.2) (layer "B.Cu") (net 6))
 (segment (start 50 47) (end 46.4 50.6) (width 0.2) (layer "B.Cu") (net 6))
 (segment (start 51 47) (end 50 47) (width 0.2) (layer "B.Cu") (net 6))
 (segment (start 39 71) (end 41 73) (width 0.2) (layer "F.Cu") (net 12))
 (segment (start 37.5 71) (end 39 71) (width 0.2) (layer "F.Cu") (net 12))
 (segment (start 22 56) (end 27 61) (width 0.2) (layer "F.Cu") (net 12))
 (via (at 37.5 71) (size 0.6) (drill 0.3) (layers "F.Cu" "B.Cu") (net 12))
 (via (at 41 73) (size 0.6) (drill 0.3) (layers "F.Cu" "B.Cu") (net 12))
 (via (at 22 56) (size 0.6) (drill 0.3) (layers "F.Cu" "B.Cu") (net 12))
 (via (at 27 61) (size 0.6) (drill 0.3) (layers "F.Cu" "B.Cu") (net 12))
 (segment (start 37 71) (end 37.5 71) (width 0.2) (layer "B.Cu") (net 12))
 (segment (start 27 61) (end 37 71) (width 0.2) (layer "B.Cu") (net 12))
 (segment (start 41 73) (end 41.32 73.32) (width 0.2) (layer "B.Cu") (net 12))
 (segment (start 21.08 47) (end 22.08 48) (width 0.2) (layer "B.Cu") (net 12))
 (segment (start 22.08 55.92) (end 22 56) (width 0.2) (layer "B.Cu") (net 12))
 (segment (start 22.08 48) (end 22.08 55.92) (width 0.2) (layer "B.Cu") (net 12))
 (segment (start 41.32 73.32) (end 41.32 76.7) (width 0.2) (layer "B.Cu") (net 12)))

